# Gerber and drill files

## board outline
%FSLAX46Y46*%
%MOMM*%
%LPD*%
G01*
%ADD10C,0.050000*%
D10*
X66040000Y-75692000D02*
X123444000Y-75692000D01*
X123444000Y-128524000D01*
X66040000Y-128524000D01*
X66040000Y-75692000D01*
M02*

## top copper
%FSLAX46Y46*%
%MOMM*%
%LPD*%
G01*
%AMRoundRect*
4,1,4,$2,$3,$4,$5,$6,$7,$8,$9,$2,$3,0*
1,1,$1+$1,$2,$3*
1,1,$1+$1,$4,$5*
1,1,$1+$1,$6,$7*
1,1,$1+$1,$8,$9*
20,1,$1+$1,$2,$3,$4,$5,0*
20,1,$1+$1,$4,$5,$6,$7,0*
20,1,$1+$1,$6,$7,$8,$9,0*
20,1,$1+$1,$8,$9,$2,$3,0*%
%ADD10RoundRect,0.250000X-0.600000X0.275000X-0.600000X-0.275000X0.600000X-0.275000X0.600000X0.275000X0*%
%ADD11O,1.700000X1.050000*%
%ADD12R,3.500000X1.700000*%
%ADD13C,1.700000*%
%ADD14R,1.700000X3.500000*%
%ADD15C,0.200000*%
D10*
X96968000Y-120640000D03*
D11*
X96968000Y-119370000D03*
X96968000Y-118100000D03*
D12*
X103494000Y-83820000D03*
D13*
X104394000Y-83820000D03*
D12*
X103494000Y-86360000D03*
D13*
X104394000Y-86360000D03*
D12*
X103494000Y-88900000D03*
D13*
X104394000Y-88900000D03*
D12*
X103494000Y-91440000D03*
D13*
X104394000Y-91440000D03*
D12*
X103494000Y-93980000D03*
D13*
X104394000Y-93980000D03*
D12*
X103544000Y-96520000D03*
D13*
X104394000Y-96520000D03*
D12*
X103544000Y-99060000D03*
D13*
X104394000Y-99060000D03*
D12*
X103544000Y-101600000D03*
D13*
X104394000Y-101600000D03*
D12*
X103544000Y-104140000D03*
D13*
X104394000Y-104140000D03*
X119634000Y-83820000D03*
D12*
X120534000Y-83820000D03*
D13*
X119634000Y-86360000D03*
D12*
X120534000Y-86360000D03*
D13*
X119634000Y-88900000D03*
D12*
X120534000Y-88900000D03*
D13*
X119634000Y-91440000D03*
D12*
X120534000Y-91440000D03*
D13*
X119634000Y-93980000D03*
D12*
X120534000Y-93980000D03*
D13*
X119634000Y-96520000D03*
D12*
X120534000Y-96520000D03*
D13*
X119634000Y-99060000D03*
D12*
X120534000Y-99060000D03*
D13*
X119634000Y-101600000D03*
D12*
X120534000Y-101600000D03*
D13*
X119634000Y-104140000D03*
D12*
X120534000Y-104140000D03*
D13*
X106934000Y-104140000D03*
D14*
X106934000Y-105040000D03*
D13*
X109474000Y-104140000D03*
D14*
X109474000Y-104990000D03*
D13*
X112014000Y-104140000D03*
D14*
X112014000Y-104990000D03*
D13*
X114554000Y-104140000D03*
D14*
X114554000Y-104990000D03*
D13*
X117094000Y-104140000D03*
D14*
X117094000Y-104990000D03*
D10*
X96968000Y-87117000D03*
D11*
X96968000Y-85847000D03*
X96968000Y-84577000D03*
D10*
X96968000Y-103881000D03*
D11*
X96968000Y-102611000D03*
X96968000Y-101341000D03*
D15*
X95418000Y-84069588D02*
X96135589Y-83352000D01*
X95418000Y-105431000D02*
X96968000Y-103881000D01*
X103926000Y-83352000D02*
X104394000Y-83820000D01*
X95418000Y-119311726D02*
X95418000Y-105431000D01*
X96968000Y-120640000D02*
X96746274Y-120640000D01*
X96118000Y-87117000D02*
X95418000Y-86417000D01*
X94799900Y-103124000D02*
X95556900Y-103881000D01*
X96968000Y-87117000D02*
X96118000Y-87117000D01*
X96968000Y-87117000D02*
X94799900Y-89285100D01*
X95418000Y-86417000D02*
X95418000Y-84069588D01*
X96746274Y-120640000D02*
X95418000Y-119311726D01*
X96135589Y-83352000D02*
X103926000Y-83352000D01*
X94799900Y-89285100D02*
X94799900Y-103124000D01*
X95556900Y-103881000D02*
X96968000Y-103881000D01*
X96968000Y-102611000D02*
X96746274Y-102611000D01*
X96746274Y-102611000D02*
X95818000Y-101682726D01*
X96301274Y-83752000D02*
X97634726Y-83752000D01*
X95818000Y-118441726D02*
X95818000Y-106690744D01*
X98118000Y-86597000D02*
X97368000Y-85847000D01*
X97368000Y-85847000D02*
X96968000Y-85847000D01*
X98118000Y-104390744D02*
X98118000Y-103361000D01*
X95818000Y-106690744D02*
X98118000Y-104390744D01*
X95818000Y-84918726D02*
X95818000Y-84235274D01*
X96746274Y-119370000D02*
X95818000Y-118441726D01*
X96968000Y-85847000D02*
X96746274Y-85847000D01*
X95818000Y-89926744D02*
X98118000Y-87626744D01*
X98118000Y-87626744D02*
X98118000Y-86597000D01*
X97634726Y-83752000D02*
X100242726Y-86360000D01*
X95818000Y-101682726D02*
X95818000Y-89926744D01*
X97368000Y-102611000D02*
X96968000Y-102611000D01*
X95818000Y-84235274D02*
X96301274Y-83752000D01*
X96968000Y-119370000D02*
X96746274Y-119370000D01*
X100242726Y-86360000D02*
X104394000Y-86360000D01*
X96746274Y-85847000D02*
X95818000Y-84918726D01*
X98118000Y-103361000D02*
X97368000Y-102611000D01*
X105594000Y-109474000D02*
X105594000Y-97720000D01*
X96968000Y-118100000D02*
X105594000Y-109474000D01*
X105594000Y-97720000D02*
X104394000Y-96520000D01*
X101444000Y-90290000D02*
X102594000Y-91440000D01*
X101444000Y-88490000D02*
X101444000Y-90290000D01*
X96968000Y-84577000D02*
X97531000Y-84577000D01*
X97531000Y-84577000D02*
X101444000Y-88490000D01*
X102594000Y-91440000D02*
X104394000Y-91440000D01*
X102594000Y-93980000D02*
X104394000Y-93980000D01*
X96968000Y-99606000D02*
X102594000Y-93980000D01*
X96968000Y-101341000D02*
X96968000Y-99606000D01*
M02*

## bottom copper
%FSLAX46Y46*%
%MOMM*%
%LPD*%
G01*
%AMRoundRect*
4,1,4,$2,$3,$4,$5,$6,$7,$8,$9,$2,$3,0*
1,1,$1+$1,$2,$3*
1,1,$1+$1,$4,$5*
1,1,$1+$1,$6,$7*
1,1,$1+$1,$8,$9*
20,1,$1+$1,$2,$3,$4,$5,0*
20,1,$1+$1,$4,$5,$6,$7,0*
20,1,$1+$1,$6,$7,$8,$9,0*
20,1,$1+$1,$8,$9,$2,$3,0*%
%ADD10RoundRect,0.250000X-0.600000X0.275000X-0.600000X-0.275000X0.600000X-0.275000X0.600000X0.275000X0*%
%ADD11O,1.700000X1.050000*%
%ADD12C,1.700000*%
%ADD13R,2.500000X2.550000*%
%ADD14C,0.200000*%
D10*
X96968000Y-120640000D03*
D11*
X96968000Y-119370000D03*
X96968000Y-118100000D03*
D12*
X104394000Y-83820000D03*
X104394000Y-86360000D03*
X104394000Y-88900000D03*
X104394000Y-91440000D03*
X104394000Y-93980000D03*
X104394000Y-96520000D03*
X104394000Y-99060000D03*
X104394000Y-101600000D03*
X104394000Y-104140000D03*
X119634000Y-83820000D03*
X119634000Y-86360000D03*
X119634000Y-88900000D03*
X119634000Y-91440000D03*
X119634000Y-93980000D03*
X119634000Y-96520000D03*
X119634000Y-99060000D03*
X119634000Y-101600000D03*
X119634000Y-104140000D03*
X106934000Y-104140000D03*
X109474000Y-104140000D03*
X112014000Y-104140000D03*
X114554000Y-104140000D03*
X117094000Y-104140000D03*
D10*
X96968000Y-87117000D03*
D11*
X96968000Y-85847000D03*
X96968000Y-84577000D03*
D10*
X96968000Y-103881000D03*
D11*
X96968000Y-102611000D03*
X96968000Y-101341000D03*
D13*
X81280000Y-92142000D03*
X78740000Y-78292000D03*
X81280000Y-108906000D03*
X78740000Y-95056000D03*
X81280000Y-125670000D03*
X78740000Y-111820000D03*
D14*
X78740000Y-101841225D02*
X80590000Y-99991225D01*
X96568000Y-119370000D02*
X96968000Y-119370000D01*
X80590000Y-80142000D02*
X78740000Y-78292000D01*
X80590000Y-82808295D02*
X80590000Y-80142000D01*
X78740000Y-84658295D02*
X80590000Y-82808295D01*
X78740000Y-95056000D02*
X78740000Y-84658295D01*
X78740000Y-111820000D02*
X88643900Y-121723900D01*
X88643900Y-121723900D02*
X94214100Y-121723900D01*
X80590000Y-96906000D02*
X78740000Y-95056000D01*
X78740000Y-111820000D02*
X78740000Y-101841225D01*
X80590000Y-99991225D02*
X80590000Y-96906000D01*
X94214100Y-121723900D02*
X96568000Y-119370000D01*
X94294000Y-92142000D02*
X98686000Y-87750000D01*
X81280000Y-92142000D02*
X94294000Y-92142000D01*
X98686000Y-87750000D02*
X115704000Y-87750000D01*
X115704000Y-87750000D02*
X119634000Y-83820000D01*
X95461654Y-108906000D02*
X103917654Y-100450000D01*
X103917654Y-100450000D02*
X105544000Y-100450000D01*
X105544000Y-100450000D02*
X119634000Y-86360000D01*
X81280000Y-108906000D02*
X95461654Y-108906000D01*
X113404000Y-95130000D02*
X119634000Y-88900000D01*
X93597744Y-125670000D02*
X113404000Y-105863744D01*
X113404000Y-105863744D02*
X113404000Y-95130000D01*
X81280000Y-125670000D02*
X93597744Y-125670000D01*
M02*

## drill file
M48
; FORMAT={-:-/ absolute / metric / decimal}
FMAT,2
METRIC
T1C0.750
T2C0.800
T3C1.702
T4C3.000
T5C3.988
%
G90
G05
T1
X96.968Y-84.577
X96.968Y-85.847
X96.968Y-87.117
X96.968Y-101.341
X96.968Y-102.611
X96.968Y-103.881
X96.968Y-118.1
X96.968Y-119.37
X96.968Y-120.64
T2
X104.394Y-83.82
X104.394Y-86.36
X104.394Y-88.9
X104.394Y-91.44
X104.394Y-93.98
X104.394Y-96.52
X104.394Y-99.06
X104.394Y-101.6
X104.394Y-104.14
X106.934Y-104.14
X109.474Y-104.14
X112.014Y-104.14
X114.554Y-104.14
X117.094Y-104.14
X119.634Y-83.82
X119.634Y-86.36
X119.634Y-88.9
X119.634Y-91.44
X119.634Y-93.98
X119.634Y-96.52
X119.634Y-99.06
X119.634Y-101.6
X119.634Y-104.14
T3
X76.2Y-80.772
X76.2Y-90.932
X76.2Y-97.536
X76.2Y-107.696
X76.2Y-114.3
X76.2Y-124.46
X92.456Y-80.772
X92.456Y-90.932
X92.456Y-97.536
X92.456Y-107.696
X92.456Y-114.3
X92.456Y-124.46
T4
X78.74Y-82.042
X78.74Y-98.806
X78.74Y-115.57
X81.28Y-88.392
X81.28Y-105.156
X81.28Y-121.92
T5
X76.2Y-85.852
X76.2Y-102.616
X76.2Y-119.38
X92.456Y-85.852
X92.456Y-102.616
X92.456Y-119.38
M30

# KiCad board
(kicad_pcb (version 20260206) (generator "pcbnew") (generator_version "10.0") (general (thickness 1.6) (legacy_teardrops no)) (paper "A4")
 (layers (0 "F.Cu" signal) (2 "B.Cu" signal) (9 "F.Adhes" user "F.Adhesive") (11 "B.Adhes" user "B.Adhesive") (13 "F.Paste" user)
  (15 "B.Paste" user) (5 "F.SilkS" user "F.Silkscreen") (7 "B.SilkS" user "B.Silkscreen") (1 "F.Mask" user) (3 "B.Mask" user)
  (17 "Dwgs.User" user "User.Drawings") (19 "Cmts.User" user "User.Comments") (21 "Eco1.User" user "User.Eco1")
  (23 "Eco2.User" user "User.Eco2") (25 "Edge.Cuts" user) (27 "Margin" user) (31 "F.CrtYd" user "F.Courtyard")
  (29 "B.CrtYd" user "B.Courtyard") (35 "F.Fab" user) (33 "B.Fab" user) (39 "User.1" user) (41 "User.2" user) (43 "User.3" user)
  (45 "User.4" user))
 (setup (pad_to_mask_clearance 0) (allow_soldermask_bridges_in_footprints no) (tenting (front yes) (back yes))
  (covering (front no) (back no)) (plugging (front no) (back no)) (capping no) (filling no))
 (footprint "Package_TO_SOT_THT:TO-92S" (layer "F.Cu") (at 96.968 120.64 90)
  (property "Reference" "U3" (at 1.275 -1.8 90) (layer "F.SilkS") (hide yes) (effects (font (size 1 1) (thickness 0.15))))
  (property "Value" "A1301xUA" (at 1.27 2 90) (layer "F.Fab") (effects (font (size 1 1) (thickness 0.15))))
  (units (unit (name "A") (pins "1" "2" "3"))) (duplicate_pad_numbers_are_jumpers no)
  (pad "1" thru_hole roundrect (at 0 0 270) (size 1.05 1.7) (drill 0.75) (layers "*.Cu" "*.Mask") (remove_unused_layers no)
   (roundrect_rratio 0.2380952381) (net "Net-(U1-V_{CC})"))
  (pad "2" thru_hole oval (at 1.27 0 270) (size 1.05 1.7) (drill 0.75) (layers "*.Cu" "*.Mask") (remove_unused_layers no)
   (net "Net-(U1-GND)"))
  (pad "3" thru_hole oval (at 2.54 0 270) (size 1.05 1.7) (drill 0.75) (layers "*.Cu" "*.Mask") (remove_unused_layers no)
   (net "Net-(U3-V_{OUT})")))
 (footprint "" (layer "F.Cu") (at 92.456 119.38)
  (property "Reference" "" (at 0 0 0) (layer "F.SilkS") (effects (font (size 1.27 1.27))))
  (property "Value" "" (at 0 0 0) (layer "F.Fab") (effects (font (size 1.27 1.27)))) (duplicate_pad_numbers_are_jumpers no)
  (pad "" np_thru_hole circle (at 0 0 270) (size 3.9878 3.9878) (drill 3.9878) (layers "*.Cu" "*.Mask")))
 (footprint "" (layer "F.Cu") (at 92.456 90.932)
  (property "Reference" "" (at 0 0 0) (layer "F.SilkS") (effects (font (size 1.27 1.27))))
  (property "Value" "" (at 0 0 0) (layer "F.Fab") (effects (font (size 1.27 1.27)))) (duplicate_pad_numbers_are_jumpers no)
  (pad "" np_thru_hole circle (at 0 0 270) (size 1.7018 1.7018) (drill 1.7018) (layers "*.Cu" "*.Mask")))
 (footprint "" (layer "F.Cu") (at 92.456 107.696)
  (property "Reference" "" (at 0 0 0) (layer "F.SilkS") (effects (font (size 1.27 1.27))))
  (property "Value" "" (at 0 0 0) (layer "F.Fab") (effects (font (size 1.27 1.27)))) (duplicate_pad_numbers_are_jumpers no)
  (pad "" np_thru_hole circle (at 0 0 270) (size 1.7018 1.7018) (drill 1.7018) (layers "*.Cu" "*.Mask")))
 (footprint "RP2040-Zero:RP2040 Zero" (layer "F.Cu") (at 101.854 106.807)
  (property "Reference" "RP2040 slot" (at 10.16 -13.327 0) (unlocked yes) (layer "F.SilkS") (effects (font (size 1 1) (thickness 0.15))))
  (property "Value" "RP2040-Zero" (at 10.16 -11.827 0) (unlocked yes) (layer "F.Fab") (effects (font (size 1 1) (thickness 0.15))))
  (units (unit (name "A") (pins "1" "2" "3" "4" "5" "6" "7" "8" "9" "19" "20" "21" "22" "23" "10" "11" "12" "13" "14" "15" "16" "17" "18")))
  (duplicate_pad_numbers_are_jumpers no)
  (pad "1" smd rect (at 1.64 -22.987) (size 3.5 1.7) (layers "F.Cu" "F.Mask") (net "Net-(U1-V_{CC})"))
  (pad "1" thru_hole circle (at 2.54 -22.987) (size 1.7 1.7) (drill 0.8) (layers "*.Cu" "*.Mask") (remove_unused_layers no)
   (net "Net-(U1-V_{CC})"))
  (pad "2" smd rect (at 1.64 -20.447) (size 3.5 1.7) (layers "F.Cu" "F.Mask") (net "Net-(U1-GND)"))
  (pad "2" thru_hole circle (at 2.54 -20.447) (size 1.7 1.7) (drill 0.8) (layers "*.Cu" "*.Mask") (remove_unused_layers no)
   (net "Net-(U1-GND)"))
  (pad "3" smd rect (at 1.64 -17.907) (size 3.5 1.7) (layers "F.Cu" "F.Mask") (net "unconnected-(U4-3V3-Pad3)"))
  (pad "3" thru_hole circle (at 2.54 -17.907) (size 1.7 1.7) (drill 0.8) (layers "*.Cu" "*.Mask") (remove_unused_layers no)
   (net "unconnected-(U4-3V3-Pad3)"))
  (pad "4" smd rect (at 1.64 -15.367) (size 3.5 1.7) (layers "F.Cu" "F.Mask") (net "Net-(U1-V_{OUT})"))
  (pad "4" thru_hole circle (at 2.54 -15.367) (size 1.7 1.7) (drill 0.8) (layers "*.Cu" "*.Mask") (remove_unused_layers no)
   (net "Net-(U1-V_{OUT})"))
  (pad "5" smd rect (at 1.64 -12.827) (size 3.5 1.7) (layers "F.Cu" "F.Mask") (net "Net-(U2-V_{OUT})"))
  (pad "5" thru_hole circle (at 2.54 -12.827) (size 1.7 1.7) (drill 0.8) (layers "*.Cu" "*.Mask") (remove_unused_layers no)
   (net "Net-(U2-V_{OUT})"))
  (pad "6" smd rect (at 1.69 -10.287) (size 3.5 1.7) (layers "F.Cu" "F.Mask") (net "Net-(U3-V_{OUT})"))
  (pad "6" thru_hole circle (at 2.54 -10.287) (size 1.7 1.7) (drill 0.8) (layers "*.Cu" "*.Mask") (remove_unused_layers no)
   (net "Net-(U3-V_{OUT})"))
  (pad "7" smd rect (at 1.69 -7.747) (size 3.5 1.7) (layers "F.Cu" "F.Mask") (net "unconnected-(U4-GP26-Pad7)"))
  (pad "7" thru_hole circle (at 2.54 -7.747) (size 1.7 1.7) (drill 0.8) (layers "*.Cu" "*.Mask") (remove_unused_layers no)
   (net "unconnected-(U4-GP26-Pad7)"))
  (pad "8" smd rect (at 1.69 -5.207) (size 3.5 1.7) (layers "F.Cu" "F.Mask") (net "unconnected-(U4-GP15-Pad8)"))
  (pad "8" thru_hole circle (at 2.54 -5.207) (size 1.7 1.7) (drill 0.8) (layers "*.Cu" "*.Mask") (remove_unused_layers no)
   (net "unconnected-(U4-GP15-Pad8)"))
  (pad "9" smd rect (at 1.69 -2.667) (size 3.5 1.7) (layers "F.Cu" "F.Mask") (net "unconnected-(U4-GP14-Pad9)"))
  (pad "9" thru_hole circle (at 2.54 -2.667) (size 1.7 1.7) (drill 0.8) (layers "*.Cu" "*.Mask") (remove_unused_layers no)
   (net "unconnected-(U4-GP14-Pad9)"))
  (pad "10" thru_hole circle (at 17.78 -22.987) (size 1.7 1.7) (drill 0.8) (layers "*.Cu" "*.Mask") (remove_unused_layers no)
   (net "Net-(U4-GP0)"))
  (pad "10" smd rect (at 18.68 -22.987) (size 3.5 1.7) (layers "F.Cu" "F.Mask") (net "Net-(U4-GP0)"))
  (pad "11" thru_hole circle (at 17.78 -20.447) (size 1.7 1.7) (drill 0.8) (layers "*.Cu" "*.Mask") (remove_unused_layers no)
   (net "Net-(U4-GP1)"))
  (pad "11" smd rect (at 18.68 -20.447) (size 3.5 1.7) (layers "F.Cu" "F.Mask") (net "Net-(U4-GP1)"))
  (pad "12" thru_hole circle (at 17.78 -17.907) (size 1.7 1.7) (drill 0.8) (layers "*.Cu" "*.Mask") (remove_unused_layers no)
   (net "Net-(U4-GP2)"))
  (pad "12" smd rect (at 18.68 -17.907) (size 3.5 1.7) (layers "F.Cu" "F.Mask") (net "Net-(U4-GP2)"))
  (pad "13" thru_hole circle (at 17.78 -15.367) (size 1.7 1.7) (drill 0.8) (layers "*.Cu" "*.Mask") (remove_unused_layers no)
   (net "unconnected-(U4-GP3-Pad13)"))
  (pad "13" smd rect (at 18.68 -15.367) (size 3.5 1.7) (layers "F.Cu" "F.Mask") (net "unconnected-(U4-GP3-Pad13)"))
  (pad "14" thru_hole circle (at 17.78 -12.827) (size 1.7 1.7) (drill 0.8) (layers "*.Cu" "*.Mask") (remove_unused_layers no)
   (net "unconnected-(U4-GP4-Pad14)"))
  (pad "14" smd rect (at 18.68 -12.827) (size 3.5 1.7) (layers "F.Cu" "F.Mask") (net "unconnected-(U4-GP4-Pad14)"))
  (pad "15" thru_hole circle (at 17.78 -10.287) (size 1.7 1.7) (drill 0.8) (layers "*.Cu" "*.Mask") (remove_unused_layers no)
   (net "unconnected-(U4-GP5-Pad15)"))
  (pad "15" smd rect (at 18.68 -10.287) (size 3.5 1.7) (layers "F.Cu" "F.Mask") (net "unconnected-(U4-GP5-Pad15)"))
  (pad "16" thru_hole circle (at 17.78 -7.747) (size 1.7 1.7) (drill 0.8) (layers "*.Cu" "*.Mask") (remove_unused_layers no)
   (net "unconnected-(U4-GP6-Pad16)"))
  (pad "16" smd rect (at 18.68 -7.747) (size 3.5 1.7) (layers "F.Cu" "F.Mask") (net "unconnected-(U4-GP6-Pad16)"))
  (pad "17" thru_hole circle (at 17.78 -5.207) (size 1.7 1.7) (drill 0.8) (layers "*.Cu" "*.Mask") (remove_unused_layers no)
   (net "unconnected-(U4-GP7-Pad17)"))
  (pad "17" smd rect (at 18.68 -5.207) (size 3.5 1.7) (layers "F.Cu" "F.Mask") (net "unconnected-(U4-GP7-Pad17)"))
  (pad "18" thru_hole circle (at 17.78 -2.667) (size 1.7 1.7) (drill 0.8) (layers "*.Cu" "*.Mask") (remove_unused_layers no)
   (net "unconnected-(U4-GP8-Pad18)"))
  (pad "18" smd rect (at 18.68 -2.667) (size 3.5 1.7) (layers "F.Cu" "F.Mask") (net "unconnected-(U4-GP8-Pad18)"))
  (pad "19" thru_hole circle (at 5.08 -2.667) (size 1.7 1.7) (drill 0.8) (layers "*.Cu" "*.Mask") (remove_unused_layers no)
   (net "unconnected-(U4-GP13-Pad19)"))
  (pad "19" smd rect (at 5.08 -1.767 90) (size 3.5 1.7) (layers "F.Cu" "F.Mask") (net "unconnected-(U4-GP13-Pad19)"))
  (pad "20" thru_hole circle (at 7.62 -2.667) (size 1.7 1.7) (drill 0.8) (layers "*.Cu" "*.Mask") (remove_unused_layers no)
   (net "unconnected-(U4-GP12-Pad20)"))
  (pad "20" smd rect (at 7.62 -1.817 90) (size 3.5 1.7) (layers "F.Cu" "F.Mask") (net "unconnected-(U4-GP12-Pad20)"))
  (pad "21" thru_hole circle (at 10.16 -2.667) (size 1.7 1.7) (drill 0.8) (layers "*.Cu" "*.Mask") (remove_unused_layers no)
   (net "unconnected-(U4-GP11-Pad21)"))
  (pad "21" smd rect (at 10.16 -1.817 90) (size 3.5 1.7) (layers "F.Cu" "F.Mask") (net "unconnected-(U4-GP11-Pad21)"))
  (pad "22" thru_hole circle (at 12.7 -2.667) (size 1.7 1.7) (drill 0.8) (layers "*.Cu" "*.Mask") (remove_unused_layers no)
   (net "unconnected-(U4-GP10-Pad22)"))
  (pad "22" smd rect (at 12.7 -1.817 90) (size 3.5 1.7) (layers "F.Cu" "F.Mask") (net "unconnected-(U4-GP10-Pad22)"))
  (pad "23" thru_hole circle (at 15.24 -2.667) (size 1.7 1.7) (drill 0.8) (layers "*.Cu" "*.Mask") (remove_unused_layers no)
   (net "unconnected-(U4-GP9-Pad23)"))
  (pad "23" smd rect (at 15.24 -1.817 90) (size 3.5 1.7) (layers "F.Cu" "F.Mask") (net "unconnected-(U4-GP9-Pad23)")))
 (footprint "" (layer "F.Cu") (at 92.456 114.3)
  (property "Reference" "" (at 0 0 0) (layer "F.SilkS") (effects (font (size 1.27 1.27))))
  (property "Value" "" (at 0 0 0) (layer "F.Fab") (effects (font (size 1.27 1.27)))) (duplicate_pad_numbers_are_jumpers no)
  (pad "" np_thru_hole circle (at 0 0 270) (size 1.7018 1.7018) (drill 1.7018) (layers "*.Cu" "*.Mask")))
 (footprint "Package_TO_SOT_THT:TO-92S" (layer "F.Cu") (at 96.968 87.117 90)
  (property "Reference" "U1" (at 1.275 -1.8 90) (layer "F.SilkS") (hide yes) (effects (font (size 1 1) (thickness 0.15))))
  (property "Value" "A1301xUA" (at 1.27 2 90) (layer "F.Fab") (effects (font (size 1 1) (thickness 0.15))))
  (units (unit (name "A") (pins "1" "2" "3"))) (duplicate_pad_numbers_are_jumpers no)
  (pad "1" thru_hole roundrect (at 0 0 270) (size 1.05 1.7) (drill 0.75) (layers "*.Cu" "*.Mask") (remove_unused_layers no)
   (roundrect_rratio 0.2380952381) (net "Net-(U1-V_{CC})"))
  (pad "2" thru_hole oval (at 1.27 0 270) (size 1.05 1.7) (drill 0.75) (layers "*.Cu" "*.Mask") (remove_unused_layers no)
   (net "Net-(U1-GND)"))
  (pad "3" thru_hole oval (at 2.54 0 270) (size 1.05 1.7) (drill 0.75) (layers "*.Cu" "*.Mask") (remove_unused_layers no)
   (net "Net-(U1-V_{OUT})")))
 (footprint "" (layer "F.Cu") (at 92.456 102.616)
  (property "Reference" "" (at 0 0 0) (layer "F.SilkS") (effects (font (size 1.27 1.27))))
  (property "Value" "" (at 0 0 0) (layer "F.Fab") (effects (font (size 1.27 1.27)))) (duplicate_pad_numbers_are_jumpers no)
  (pad "" np_thru_hole circle (at 0 0 270) (size 3.9878 3.9878) (drill 3.9878) (layers "*.Cu" "*.Mask")))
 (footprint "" (layer "F.Cu") (at 92.456 80.772)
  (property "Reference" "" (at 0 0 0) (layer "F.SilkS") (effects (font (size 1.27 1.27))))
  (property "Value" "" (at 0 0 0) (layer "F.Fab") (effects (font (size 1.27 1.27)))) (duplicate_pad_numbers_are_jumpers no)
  (pad "" np_thru_hole circle (at 0 0 270) (size 1.7018 1.7018) (drill 1.7018) (layers "*.Cu" "*.Mask")))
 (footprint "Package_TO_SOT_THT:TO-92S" (layer "F.Cu") (at 96.968 103.881 90)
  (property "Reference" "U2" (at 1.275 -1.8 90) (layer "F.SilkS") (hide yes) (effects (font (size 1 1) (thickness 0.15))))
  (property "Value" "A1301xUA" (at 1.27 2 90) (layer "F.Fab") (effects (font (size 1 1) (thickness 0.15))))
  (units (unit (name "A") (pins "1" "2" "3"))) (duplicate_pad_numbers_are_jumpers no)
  (pad "1" thru_hole roundrect (at 0 0 270) (size 1.05 1.7) (drill 0.75) (layers "*.Cu" "*.Mask") (remove_unused_layers no)
   (roundrect_rratio 0.2380952381) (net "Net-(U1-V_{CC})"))
  (pad "2" thru_hole oval (at 1.27 0 270) (size 1.05 1.7) (drill 0.75) (layers "*.Cu" "*.Mask") (remove_unused_layers no)
   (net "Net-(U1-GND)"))
  (pad "3" thru_hole oval (at 2.54 0 270) (size 1.05 1.7) (drill 0.75) (layers "*.Cu" "*.Mask") (remove_unused_layers no)
   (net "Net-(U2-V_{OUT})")))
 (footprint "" (layer "F.Cu") (at 92.456 85.852)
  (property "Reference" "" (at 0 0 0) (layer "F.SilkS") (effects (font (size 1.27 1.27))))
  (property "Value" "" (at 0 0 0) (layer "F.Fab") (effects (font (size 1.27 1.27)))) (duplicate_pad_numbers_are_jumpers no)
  (pad "" np_thru_hole circle (at 0 0 270) (size 3.9878 3.9878) (drill 3.9878) (layers "*.Cu" "*.Mask")))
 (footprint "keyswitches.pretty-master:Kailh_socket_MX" (layer "F.Cu") (at 76.2 85.852 -90)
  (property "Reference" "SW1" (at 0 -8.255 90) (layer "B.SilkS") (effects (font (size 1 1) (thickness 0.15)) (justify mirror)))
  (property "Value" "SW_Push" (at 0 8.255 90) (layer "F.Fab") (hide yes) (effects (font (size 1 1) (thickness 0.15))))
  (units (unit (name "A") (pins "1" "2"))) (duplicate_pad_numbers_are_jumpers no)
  (pad "" np_thru_hole circle (at -5.08 0 270) (size 1.7018 1.7018) (drill 1.7018) (layers "*.Cu" "*.Mask"))
  (pad "" np_thru_hole circle (at -3.81 -2.54 270) (size 3 3) (drill 3) (layers "*.Cu" "*.Mask"))
  (pad "" np_thru_hole circle (at 0 0 270) (size 3.9878 3.9878) (drill 3.9878) (layers "*.Cu" "*.Mask"))
  (pad "" np_thru_hole circle (at 2.54 -5.08 270) (size 3 3) (drill 3) (layers "*.Cu" "*.Mask"))
  (pad "" np_thru_hole circle (at 5.08 0 270) (size 1.7018 1.7018) (drill 1.7018) (layers "*.Cu" "*.Mask"))
  (pad "1" smd rect (at 6.29 -5.08 270) (size 2.55 2.5) (layers "B.Cu" "B.Mask" "B.Paste") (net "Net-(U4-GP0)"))
  (pad "2" smd rect (at -7.56 -2.54 270) (size 2.55 2.5) (layers "B.Cu" "B.Mask" "B.Paste") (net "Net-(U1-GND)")))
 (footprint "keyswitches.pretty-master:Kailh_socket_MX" (layer "F.Cu") (at 76.2 102.616 -90)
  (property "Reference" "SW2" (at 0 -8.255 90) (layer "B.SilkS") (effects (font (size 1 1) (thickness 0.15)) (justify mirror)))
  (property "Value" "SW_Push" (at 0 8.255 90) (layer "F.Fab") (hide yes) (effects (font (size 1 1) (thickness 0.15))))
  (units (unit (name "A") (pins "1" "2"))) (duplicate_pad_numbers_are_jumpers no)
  (pad "" np_thru_hole circle (at -5.08 0 270) (size 1.7018 1.7018) (drill 1.7018) (layers "*.Cu" "*.Mask"))
  (pad "" np_thru_hole circle (at -3.81 -2.54 270) (size 3 3) (drill 3) (layers "*.Cu" "*.Mask"))
  (pad "" np_thru_hole circle (at 0 0 270) (size 3.9878 3.9878) (drill 3.9878) (layers "*.Cu" "*.Mask"))
  (pad "" np_thru_hole circle (at 2.54 -5.08 270) (size 3 3) (drill 3) (layers "*.Cu" "*.Mask"))
  (pad "" np_thru_hole circle (at 5.08 0 270) (size 1.7018 1.7018) (drill 1.7018) (layers "*.Cu" "*.Mask"))
  (pad "1" smd rect (at 6.29 -5.08 270) (size 2.55 2.5) (layers "B.Cu" "B.Mask" "B.Paste") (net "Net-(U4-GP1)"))
  (pad "2" smd rect (at -7.56 -2.54 270) (size 2.55 2.5) (layers "B.Cu" "B.Mask" "B.Paste") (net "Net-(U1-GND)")))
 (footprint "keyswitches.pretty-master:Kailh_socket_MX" (layer "F.Cu") (at 76.2 119.38 -90)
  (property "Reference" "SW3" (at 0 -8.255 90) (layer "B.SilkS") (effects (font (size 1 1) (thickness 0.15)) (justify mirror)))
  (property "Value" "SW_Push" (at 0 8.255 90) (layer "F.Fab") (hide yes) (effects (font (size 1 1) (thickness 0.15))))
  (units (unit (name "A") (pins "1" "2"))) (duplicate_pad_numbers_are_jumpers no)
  (pad "" np_thru_hole circle (at -5.08 0 270) (size 1.7018 1.7018) (drill 1.7018) (layers "*.Cu" "*.Mask"))
  (pad "" np_thru_hole circle (at -3.81 -2.54 270) (size 3 3) (drill 3) (layers "*.Cu" "*.Mask"))
  (pad "" np_thru_hole circle (at 0 0 270) (size 3.9878 3.9878) (drill 3.9878) (layers "*.Cu" "*.Mask"))
  (pad "" np_thru_hole circle (at 2.54 -5.08 270) (size 3 3) (drill 3) (layers "*.Cu" "*.Mask"))
  (pad "" np_thru_hole circle (at 5.08 0 270) (size 1.7018 1.7018) (drill 1.7018) (layers "*.Cu" "*.Mask"))
  (pad "1" smd rect (at 6.29 -5.08 270) (size 2.55 2.5) (layers "B.Cu" "B.Mask" "B.Paste") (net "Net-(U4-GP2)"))
  (pad "2" smd rect (at -7.56 -2.54 270) (size 2.55 2.5) (layers "B.Cu" "B.Mask" "B.Paste") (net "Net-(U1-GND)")))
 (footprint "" (layer "F.Cu") (at 92.456 124.46)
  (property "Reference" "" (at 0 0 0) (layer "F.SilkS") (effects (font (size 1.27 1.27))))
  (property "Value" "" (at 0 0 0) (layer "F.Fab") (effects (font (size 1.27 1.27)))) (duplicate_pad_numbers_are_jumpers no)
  (pad "" np_thru_hole circle (at 0 0 270) (size 1.7018 1.7018) (drill 1.7018) (layers "*.Cu" "*.Mask")))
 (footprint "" (layer "F.Cu") (at 92.456 97.536)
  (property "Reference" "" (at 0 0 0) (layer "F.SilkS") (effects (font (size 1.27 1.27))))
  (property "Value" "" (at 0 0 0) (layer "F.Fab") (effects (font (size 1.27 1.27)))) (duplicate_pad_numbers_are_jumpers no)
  (pad "" np_thru_hole circle (at 0 0 270) (size 1.7018 1.7018) (drill 1.7018) (layers "*.Cu" "*.Mask")))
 (gr_rect (start 66.04 75.692) (end 123.444 128.524) (stroke (width 0.05) (type default)) (fill no) (layer "Edge.Cuts"))
 (segment (start 95.418 84.069588) (end 96.135589 83.352) (width 0.2) (layer "F.Cu") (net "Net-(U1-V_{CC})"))
 (segment (start 95.418 105.431) (end 96.968 103.881) (width 0.2) (layer "F.Cu") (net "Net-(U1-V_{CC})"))
 (segment (start 103.926 83.352) (end 104.394 83.82) (width 0.2) (layer "F.Cu") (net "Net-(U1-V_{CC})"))
 (segment (start 95.418 119.311726) (end 95.418 105.431) (width 0.2) (layer "F.Cu") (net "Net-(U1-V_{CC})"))
 (segment (start 96.968 120.64) (end 96.746274 120.64) (width 0.2) (layer "F.Cu") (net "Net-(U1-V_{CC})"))
 (segment (start 96.118 87.117) (end 95.418 86.417) (width 0.2) (layer "F.Cu") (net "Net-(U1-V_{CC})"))
 (segment (start 94.7999 103.124) (end 95.5569 103.881) (width 0.2) (layer "F.Cu") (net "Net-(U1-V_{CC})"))
 (segment (start 96.968 87.117) (end 96.118 87.117) (width 0.2) (layer "F.Cu") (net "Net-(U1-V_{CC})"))
 (segment (start 96.968 87.117) (end 94.7999 89.2851) (width 0.2) (layer "F.Cu") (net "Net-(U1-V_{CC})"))
 (segment (start 95.418 86.417) (end 95.418 84.069588) (width 0.2) (layer "F.Cu") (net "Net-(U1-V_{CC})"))
 (segment (start 96.746274 120.64) (end 95.418 119.311726) (width 0.2) (layer "F.Cu") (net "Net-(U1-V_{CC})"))
 (segment (start 96.135589 83.352) (end 103.926 83.352) (width 0.2) (layer "F.Cu") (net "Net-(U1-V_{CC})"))
 (segment (start 94.7999 89.2851) (end 94.7999 103.124) (width 0.2) (layer "F.Cu") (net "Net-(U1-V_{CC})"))
 (segment (start 95.5569 103.881) (end 96.968 103.881) (width 0.2) (layer "F.Cu") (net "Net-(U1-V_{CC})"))
 (segment (start 96.968 102.611) (end 96.746274 102.611) (width 0.2) (layer "F.Cu") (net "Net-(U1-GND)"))
 (segment (start 96.746274 102.611) (end 95.818 101.682726) (width 0.2) (layer "F.Cu") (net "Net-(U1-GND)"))
 (segment (start 96.301274 83.752) (end 97.634726 83.752) (width 0.2) (layer "F.Cu") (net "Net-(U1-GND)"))
 (segment (start 95.818 118.441726) (end 95.818 106.690744) (width 0.2) (layer "F.Cu") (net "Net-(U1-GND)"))
 (segment (start 98.118 86.597) (end 97.368 85.847) (width 0.2) (layer "F.Cu") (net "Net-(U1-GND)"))
 (segment (start 97.368 85.847) (end 96.968 85.847) (width 0.2) (layer "F.Cu") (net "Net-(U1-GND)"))
 (segment (start 98.118 104.390744) (end 98.118 103.361) (width 0.2) (layer "F.Cu") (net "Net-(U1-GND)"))
 (segment (start 95.818 106.690744) (end 98.118 104.390744) (width 0.2) (layer "F.Cu") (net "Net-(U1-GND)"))
 (segment (start 95.818 84.918726) (end 95.818 84.235274) (width 0.2) (layer "F.Cu") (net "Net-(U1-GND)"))
 (segment (start 96.746274 119.37) (end 95.818 118.441726) (width 0.2) (layer "F.Cu") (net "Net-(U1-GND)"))
 (segment (start 96.968 85.847) (end 96.746274 85.847) (width 0.2) (layer "F.Cu") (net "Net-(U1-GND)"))
 (segment (start 95.818 89.926744) (end 98.118 87.626744) (width 0.2) (layer "F.Cu") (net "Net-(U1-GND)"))
 (segment (start 98.118 87.626744) (end 98.118 86.597) (width 0.2) (layer "F.Cu") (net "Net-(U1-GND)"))
 (segment (start 97.634726 83.752) (end 100.242726 86.36) (width 0.2) (layer "F.Cu") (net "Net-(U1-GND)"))
 (segment (start 95.818 101.682726) (end 95.818 89.926744) (width 0.2) (layer "F.Cu") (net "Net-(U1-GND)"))
 (segment (start 97.368 102.611) (end 96.968 102.611) (width 0.2) (layer "F.Cu") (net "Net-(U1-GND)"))
 (segment (start 95.818 84.235274) (end 96.301274 83.752) (width 0.2) (layer "F.Cu") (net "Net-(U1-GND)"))
 (segment (start 96.968 119.37) (end 96.746274 119.37) (width 0.2) (layer "F.Cu") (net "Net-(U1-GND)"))
 (segment (start 100.242726 86.36) (end 104.394 86.36) (width 0.2) (layer "F.Cu") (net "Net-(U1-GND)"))
 (segment (start 96.746274 85.847) (end 95.818 84.918726) (width 0.2) (layer "F.Cu") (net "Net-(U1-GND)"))
 (segment (start 98.118 103.361) (end 97.368 102.611) (width 0.2) (layer "F.Cu") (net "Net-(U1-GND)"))
 (segment (start 78.74 101.841225) (end 80.59 99.991225) (width 0.2) (layer "B.Cu") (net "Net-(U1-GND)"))
 (segment (start 96.568 119.37) (end 96.968 119.37) (width 0.2) (layer "B.Cu") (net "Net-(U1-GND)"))
 (segment (start 80.59 80.142) (end 78.74 78.292) (width 0.2) (layer "B.Cu") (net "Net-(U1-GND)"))
 (segment (start 80.59 82.808295) (end 80.59 80.142) (width 0.2) (layer "B.Cu") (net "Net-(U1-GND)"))
 (segment (start 78.74 84.658295) (end 80.59 82.808295) (width 0.2) (layer "B.Cu") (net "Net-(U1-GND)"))
 (segment (start 78.74 95.056) (end 78.74 84.658295) (width 0.2) (layer "B.Cu") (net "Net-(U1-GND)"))
 (segment (start 78.74 111.82) (end 88.6439 121.7239) (width 0.2) (layer "B.Cu") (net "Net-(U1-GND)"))
 (segment (start 88.6439 121.7239) (end 94.2141 121.7239) (width 0.2) (layer "B.Cu") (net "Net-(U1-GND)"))
 (segment (start 80.59 96.906) (end 78.74 95.056) (width 0.2) (layer "B.Cu") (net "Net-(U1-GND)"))
 (segment (start 78.74 111.82) (end 78.74 101.841225) (width 0.2) (layer "B.Cu") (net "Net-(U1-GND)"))
 (segment (start 80.59 99.991225) (end 80.59 96.906) (width 0.2) (layer "B.Cu") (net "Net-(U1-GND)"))
 (segment (start 94.2141 121.7239) (end 96.568 119.37) (width 0.2) (layer "B.Cu") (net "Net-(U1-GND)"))
 (segment (start 105.594 109.474) (end 105.594 97.72) (width 0.2) (layer "F.Cu") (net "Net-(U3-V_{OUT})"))
 (segment (start 96.968 118.1) (end 105.594 109.474) (width 0.2) (layer "F.Cu") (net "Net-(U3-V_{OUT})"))
 (segment (start 105.594 97.72) (end 104.394 96.52) (width 0.2) (layer "F.Cu") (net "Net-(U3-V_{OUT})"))
 (segment (start 101.444 90.29) (end 102.594 91.44) (width 0.2) (layer "F.Cu") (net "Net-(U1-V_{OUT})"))
 (segment (start 101.444 88.49) (end 101.444 90.29) (width 0.2) (layer "F.Cu") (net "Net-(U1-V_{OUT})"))
 (segment (start 96.968 84.577) (end 97.531 84.577) (width 0.2) (layer "F.Cu") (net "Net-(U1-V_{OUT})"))
 (segment (start 97.531 84.577) (end 101.444 88.49) (width 0.2) (layer "F.Cu") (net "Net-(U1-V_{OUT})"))
 (segment (start 102.594 91.44) (end 104.394 91.44) (width 0.2) (layer "F.Cu") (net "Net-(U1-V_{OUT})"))
 (segment (start 102.594 93.98) (end 104.394 93.98) (width 0.2) (layer "F.Cu") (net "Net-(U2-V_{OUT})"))
 (segment (start 96.968 99.606) (end 102.594 93.98) (width 0.2) (layer "F.Cu") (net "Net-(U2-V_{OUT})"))
 (segment (start 96.968 101.341) (end 96.968 99.606) (width 0.2) (layer "F.Cu") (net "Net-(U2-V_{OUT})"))
 (segment (start 94.294 92.142) (end 98.686 87.75) (width 0.2) (layer "B.Cu") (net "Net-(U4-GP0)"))
 (segment (start 81.28 92.142) (end 94.294 92.142) (width 0.2) (layer "B.Cu") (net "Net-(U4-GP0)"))
 (segment (start 98.686 87.75) (end 115.704 87.75) (width 0.2) (layer "B.Cu") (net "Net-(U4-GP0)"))
 (segment (start 115.704 87.75) (end 119.634 83.82) (width 0.2) (layer "B.Cu") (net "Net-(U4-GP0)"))
 (segment (start 95.461654 108.906) (end 103.917654 100.45) (width 0.2) (layer "B.Cu") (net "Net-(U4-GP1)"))
 (segment (start 103.917654 100.45) (end 105.544 100.45) (width 0.2) (layer "B.Cu") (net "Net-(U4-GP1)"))
 (segment (start 105.544 100.45) (end 119.634 86.36) (width 0.2) (layer "B.Cu") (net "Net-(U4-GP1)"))
 (segment (start 81.28 108.906) (end 95.461654 108.906) (width 0.2) (layer "B.Cu") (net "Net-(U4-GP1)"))
 (segment (start 113.404 95.13) (end 119.634 88.9) (width 0.2) (layer "B.Cu") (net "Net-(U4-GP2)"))
 (segment (start 93.597744 125.67) (end 113.404 105.863744) (width 0.2) (layer "B.Cu") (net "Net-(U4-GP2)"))
 (segment (start 113.404 105.863744) (end 113.404 95.13) (width 0.2) (layer "B.Cu") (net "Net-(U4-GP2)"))
 (segment (start 81.28 125.67) (end 93.597744 125.67) (width 0.2) (layer "B.Cu") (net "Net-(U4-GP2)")))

